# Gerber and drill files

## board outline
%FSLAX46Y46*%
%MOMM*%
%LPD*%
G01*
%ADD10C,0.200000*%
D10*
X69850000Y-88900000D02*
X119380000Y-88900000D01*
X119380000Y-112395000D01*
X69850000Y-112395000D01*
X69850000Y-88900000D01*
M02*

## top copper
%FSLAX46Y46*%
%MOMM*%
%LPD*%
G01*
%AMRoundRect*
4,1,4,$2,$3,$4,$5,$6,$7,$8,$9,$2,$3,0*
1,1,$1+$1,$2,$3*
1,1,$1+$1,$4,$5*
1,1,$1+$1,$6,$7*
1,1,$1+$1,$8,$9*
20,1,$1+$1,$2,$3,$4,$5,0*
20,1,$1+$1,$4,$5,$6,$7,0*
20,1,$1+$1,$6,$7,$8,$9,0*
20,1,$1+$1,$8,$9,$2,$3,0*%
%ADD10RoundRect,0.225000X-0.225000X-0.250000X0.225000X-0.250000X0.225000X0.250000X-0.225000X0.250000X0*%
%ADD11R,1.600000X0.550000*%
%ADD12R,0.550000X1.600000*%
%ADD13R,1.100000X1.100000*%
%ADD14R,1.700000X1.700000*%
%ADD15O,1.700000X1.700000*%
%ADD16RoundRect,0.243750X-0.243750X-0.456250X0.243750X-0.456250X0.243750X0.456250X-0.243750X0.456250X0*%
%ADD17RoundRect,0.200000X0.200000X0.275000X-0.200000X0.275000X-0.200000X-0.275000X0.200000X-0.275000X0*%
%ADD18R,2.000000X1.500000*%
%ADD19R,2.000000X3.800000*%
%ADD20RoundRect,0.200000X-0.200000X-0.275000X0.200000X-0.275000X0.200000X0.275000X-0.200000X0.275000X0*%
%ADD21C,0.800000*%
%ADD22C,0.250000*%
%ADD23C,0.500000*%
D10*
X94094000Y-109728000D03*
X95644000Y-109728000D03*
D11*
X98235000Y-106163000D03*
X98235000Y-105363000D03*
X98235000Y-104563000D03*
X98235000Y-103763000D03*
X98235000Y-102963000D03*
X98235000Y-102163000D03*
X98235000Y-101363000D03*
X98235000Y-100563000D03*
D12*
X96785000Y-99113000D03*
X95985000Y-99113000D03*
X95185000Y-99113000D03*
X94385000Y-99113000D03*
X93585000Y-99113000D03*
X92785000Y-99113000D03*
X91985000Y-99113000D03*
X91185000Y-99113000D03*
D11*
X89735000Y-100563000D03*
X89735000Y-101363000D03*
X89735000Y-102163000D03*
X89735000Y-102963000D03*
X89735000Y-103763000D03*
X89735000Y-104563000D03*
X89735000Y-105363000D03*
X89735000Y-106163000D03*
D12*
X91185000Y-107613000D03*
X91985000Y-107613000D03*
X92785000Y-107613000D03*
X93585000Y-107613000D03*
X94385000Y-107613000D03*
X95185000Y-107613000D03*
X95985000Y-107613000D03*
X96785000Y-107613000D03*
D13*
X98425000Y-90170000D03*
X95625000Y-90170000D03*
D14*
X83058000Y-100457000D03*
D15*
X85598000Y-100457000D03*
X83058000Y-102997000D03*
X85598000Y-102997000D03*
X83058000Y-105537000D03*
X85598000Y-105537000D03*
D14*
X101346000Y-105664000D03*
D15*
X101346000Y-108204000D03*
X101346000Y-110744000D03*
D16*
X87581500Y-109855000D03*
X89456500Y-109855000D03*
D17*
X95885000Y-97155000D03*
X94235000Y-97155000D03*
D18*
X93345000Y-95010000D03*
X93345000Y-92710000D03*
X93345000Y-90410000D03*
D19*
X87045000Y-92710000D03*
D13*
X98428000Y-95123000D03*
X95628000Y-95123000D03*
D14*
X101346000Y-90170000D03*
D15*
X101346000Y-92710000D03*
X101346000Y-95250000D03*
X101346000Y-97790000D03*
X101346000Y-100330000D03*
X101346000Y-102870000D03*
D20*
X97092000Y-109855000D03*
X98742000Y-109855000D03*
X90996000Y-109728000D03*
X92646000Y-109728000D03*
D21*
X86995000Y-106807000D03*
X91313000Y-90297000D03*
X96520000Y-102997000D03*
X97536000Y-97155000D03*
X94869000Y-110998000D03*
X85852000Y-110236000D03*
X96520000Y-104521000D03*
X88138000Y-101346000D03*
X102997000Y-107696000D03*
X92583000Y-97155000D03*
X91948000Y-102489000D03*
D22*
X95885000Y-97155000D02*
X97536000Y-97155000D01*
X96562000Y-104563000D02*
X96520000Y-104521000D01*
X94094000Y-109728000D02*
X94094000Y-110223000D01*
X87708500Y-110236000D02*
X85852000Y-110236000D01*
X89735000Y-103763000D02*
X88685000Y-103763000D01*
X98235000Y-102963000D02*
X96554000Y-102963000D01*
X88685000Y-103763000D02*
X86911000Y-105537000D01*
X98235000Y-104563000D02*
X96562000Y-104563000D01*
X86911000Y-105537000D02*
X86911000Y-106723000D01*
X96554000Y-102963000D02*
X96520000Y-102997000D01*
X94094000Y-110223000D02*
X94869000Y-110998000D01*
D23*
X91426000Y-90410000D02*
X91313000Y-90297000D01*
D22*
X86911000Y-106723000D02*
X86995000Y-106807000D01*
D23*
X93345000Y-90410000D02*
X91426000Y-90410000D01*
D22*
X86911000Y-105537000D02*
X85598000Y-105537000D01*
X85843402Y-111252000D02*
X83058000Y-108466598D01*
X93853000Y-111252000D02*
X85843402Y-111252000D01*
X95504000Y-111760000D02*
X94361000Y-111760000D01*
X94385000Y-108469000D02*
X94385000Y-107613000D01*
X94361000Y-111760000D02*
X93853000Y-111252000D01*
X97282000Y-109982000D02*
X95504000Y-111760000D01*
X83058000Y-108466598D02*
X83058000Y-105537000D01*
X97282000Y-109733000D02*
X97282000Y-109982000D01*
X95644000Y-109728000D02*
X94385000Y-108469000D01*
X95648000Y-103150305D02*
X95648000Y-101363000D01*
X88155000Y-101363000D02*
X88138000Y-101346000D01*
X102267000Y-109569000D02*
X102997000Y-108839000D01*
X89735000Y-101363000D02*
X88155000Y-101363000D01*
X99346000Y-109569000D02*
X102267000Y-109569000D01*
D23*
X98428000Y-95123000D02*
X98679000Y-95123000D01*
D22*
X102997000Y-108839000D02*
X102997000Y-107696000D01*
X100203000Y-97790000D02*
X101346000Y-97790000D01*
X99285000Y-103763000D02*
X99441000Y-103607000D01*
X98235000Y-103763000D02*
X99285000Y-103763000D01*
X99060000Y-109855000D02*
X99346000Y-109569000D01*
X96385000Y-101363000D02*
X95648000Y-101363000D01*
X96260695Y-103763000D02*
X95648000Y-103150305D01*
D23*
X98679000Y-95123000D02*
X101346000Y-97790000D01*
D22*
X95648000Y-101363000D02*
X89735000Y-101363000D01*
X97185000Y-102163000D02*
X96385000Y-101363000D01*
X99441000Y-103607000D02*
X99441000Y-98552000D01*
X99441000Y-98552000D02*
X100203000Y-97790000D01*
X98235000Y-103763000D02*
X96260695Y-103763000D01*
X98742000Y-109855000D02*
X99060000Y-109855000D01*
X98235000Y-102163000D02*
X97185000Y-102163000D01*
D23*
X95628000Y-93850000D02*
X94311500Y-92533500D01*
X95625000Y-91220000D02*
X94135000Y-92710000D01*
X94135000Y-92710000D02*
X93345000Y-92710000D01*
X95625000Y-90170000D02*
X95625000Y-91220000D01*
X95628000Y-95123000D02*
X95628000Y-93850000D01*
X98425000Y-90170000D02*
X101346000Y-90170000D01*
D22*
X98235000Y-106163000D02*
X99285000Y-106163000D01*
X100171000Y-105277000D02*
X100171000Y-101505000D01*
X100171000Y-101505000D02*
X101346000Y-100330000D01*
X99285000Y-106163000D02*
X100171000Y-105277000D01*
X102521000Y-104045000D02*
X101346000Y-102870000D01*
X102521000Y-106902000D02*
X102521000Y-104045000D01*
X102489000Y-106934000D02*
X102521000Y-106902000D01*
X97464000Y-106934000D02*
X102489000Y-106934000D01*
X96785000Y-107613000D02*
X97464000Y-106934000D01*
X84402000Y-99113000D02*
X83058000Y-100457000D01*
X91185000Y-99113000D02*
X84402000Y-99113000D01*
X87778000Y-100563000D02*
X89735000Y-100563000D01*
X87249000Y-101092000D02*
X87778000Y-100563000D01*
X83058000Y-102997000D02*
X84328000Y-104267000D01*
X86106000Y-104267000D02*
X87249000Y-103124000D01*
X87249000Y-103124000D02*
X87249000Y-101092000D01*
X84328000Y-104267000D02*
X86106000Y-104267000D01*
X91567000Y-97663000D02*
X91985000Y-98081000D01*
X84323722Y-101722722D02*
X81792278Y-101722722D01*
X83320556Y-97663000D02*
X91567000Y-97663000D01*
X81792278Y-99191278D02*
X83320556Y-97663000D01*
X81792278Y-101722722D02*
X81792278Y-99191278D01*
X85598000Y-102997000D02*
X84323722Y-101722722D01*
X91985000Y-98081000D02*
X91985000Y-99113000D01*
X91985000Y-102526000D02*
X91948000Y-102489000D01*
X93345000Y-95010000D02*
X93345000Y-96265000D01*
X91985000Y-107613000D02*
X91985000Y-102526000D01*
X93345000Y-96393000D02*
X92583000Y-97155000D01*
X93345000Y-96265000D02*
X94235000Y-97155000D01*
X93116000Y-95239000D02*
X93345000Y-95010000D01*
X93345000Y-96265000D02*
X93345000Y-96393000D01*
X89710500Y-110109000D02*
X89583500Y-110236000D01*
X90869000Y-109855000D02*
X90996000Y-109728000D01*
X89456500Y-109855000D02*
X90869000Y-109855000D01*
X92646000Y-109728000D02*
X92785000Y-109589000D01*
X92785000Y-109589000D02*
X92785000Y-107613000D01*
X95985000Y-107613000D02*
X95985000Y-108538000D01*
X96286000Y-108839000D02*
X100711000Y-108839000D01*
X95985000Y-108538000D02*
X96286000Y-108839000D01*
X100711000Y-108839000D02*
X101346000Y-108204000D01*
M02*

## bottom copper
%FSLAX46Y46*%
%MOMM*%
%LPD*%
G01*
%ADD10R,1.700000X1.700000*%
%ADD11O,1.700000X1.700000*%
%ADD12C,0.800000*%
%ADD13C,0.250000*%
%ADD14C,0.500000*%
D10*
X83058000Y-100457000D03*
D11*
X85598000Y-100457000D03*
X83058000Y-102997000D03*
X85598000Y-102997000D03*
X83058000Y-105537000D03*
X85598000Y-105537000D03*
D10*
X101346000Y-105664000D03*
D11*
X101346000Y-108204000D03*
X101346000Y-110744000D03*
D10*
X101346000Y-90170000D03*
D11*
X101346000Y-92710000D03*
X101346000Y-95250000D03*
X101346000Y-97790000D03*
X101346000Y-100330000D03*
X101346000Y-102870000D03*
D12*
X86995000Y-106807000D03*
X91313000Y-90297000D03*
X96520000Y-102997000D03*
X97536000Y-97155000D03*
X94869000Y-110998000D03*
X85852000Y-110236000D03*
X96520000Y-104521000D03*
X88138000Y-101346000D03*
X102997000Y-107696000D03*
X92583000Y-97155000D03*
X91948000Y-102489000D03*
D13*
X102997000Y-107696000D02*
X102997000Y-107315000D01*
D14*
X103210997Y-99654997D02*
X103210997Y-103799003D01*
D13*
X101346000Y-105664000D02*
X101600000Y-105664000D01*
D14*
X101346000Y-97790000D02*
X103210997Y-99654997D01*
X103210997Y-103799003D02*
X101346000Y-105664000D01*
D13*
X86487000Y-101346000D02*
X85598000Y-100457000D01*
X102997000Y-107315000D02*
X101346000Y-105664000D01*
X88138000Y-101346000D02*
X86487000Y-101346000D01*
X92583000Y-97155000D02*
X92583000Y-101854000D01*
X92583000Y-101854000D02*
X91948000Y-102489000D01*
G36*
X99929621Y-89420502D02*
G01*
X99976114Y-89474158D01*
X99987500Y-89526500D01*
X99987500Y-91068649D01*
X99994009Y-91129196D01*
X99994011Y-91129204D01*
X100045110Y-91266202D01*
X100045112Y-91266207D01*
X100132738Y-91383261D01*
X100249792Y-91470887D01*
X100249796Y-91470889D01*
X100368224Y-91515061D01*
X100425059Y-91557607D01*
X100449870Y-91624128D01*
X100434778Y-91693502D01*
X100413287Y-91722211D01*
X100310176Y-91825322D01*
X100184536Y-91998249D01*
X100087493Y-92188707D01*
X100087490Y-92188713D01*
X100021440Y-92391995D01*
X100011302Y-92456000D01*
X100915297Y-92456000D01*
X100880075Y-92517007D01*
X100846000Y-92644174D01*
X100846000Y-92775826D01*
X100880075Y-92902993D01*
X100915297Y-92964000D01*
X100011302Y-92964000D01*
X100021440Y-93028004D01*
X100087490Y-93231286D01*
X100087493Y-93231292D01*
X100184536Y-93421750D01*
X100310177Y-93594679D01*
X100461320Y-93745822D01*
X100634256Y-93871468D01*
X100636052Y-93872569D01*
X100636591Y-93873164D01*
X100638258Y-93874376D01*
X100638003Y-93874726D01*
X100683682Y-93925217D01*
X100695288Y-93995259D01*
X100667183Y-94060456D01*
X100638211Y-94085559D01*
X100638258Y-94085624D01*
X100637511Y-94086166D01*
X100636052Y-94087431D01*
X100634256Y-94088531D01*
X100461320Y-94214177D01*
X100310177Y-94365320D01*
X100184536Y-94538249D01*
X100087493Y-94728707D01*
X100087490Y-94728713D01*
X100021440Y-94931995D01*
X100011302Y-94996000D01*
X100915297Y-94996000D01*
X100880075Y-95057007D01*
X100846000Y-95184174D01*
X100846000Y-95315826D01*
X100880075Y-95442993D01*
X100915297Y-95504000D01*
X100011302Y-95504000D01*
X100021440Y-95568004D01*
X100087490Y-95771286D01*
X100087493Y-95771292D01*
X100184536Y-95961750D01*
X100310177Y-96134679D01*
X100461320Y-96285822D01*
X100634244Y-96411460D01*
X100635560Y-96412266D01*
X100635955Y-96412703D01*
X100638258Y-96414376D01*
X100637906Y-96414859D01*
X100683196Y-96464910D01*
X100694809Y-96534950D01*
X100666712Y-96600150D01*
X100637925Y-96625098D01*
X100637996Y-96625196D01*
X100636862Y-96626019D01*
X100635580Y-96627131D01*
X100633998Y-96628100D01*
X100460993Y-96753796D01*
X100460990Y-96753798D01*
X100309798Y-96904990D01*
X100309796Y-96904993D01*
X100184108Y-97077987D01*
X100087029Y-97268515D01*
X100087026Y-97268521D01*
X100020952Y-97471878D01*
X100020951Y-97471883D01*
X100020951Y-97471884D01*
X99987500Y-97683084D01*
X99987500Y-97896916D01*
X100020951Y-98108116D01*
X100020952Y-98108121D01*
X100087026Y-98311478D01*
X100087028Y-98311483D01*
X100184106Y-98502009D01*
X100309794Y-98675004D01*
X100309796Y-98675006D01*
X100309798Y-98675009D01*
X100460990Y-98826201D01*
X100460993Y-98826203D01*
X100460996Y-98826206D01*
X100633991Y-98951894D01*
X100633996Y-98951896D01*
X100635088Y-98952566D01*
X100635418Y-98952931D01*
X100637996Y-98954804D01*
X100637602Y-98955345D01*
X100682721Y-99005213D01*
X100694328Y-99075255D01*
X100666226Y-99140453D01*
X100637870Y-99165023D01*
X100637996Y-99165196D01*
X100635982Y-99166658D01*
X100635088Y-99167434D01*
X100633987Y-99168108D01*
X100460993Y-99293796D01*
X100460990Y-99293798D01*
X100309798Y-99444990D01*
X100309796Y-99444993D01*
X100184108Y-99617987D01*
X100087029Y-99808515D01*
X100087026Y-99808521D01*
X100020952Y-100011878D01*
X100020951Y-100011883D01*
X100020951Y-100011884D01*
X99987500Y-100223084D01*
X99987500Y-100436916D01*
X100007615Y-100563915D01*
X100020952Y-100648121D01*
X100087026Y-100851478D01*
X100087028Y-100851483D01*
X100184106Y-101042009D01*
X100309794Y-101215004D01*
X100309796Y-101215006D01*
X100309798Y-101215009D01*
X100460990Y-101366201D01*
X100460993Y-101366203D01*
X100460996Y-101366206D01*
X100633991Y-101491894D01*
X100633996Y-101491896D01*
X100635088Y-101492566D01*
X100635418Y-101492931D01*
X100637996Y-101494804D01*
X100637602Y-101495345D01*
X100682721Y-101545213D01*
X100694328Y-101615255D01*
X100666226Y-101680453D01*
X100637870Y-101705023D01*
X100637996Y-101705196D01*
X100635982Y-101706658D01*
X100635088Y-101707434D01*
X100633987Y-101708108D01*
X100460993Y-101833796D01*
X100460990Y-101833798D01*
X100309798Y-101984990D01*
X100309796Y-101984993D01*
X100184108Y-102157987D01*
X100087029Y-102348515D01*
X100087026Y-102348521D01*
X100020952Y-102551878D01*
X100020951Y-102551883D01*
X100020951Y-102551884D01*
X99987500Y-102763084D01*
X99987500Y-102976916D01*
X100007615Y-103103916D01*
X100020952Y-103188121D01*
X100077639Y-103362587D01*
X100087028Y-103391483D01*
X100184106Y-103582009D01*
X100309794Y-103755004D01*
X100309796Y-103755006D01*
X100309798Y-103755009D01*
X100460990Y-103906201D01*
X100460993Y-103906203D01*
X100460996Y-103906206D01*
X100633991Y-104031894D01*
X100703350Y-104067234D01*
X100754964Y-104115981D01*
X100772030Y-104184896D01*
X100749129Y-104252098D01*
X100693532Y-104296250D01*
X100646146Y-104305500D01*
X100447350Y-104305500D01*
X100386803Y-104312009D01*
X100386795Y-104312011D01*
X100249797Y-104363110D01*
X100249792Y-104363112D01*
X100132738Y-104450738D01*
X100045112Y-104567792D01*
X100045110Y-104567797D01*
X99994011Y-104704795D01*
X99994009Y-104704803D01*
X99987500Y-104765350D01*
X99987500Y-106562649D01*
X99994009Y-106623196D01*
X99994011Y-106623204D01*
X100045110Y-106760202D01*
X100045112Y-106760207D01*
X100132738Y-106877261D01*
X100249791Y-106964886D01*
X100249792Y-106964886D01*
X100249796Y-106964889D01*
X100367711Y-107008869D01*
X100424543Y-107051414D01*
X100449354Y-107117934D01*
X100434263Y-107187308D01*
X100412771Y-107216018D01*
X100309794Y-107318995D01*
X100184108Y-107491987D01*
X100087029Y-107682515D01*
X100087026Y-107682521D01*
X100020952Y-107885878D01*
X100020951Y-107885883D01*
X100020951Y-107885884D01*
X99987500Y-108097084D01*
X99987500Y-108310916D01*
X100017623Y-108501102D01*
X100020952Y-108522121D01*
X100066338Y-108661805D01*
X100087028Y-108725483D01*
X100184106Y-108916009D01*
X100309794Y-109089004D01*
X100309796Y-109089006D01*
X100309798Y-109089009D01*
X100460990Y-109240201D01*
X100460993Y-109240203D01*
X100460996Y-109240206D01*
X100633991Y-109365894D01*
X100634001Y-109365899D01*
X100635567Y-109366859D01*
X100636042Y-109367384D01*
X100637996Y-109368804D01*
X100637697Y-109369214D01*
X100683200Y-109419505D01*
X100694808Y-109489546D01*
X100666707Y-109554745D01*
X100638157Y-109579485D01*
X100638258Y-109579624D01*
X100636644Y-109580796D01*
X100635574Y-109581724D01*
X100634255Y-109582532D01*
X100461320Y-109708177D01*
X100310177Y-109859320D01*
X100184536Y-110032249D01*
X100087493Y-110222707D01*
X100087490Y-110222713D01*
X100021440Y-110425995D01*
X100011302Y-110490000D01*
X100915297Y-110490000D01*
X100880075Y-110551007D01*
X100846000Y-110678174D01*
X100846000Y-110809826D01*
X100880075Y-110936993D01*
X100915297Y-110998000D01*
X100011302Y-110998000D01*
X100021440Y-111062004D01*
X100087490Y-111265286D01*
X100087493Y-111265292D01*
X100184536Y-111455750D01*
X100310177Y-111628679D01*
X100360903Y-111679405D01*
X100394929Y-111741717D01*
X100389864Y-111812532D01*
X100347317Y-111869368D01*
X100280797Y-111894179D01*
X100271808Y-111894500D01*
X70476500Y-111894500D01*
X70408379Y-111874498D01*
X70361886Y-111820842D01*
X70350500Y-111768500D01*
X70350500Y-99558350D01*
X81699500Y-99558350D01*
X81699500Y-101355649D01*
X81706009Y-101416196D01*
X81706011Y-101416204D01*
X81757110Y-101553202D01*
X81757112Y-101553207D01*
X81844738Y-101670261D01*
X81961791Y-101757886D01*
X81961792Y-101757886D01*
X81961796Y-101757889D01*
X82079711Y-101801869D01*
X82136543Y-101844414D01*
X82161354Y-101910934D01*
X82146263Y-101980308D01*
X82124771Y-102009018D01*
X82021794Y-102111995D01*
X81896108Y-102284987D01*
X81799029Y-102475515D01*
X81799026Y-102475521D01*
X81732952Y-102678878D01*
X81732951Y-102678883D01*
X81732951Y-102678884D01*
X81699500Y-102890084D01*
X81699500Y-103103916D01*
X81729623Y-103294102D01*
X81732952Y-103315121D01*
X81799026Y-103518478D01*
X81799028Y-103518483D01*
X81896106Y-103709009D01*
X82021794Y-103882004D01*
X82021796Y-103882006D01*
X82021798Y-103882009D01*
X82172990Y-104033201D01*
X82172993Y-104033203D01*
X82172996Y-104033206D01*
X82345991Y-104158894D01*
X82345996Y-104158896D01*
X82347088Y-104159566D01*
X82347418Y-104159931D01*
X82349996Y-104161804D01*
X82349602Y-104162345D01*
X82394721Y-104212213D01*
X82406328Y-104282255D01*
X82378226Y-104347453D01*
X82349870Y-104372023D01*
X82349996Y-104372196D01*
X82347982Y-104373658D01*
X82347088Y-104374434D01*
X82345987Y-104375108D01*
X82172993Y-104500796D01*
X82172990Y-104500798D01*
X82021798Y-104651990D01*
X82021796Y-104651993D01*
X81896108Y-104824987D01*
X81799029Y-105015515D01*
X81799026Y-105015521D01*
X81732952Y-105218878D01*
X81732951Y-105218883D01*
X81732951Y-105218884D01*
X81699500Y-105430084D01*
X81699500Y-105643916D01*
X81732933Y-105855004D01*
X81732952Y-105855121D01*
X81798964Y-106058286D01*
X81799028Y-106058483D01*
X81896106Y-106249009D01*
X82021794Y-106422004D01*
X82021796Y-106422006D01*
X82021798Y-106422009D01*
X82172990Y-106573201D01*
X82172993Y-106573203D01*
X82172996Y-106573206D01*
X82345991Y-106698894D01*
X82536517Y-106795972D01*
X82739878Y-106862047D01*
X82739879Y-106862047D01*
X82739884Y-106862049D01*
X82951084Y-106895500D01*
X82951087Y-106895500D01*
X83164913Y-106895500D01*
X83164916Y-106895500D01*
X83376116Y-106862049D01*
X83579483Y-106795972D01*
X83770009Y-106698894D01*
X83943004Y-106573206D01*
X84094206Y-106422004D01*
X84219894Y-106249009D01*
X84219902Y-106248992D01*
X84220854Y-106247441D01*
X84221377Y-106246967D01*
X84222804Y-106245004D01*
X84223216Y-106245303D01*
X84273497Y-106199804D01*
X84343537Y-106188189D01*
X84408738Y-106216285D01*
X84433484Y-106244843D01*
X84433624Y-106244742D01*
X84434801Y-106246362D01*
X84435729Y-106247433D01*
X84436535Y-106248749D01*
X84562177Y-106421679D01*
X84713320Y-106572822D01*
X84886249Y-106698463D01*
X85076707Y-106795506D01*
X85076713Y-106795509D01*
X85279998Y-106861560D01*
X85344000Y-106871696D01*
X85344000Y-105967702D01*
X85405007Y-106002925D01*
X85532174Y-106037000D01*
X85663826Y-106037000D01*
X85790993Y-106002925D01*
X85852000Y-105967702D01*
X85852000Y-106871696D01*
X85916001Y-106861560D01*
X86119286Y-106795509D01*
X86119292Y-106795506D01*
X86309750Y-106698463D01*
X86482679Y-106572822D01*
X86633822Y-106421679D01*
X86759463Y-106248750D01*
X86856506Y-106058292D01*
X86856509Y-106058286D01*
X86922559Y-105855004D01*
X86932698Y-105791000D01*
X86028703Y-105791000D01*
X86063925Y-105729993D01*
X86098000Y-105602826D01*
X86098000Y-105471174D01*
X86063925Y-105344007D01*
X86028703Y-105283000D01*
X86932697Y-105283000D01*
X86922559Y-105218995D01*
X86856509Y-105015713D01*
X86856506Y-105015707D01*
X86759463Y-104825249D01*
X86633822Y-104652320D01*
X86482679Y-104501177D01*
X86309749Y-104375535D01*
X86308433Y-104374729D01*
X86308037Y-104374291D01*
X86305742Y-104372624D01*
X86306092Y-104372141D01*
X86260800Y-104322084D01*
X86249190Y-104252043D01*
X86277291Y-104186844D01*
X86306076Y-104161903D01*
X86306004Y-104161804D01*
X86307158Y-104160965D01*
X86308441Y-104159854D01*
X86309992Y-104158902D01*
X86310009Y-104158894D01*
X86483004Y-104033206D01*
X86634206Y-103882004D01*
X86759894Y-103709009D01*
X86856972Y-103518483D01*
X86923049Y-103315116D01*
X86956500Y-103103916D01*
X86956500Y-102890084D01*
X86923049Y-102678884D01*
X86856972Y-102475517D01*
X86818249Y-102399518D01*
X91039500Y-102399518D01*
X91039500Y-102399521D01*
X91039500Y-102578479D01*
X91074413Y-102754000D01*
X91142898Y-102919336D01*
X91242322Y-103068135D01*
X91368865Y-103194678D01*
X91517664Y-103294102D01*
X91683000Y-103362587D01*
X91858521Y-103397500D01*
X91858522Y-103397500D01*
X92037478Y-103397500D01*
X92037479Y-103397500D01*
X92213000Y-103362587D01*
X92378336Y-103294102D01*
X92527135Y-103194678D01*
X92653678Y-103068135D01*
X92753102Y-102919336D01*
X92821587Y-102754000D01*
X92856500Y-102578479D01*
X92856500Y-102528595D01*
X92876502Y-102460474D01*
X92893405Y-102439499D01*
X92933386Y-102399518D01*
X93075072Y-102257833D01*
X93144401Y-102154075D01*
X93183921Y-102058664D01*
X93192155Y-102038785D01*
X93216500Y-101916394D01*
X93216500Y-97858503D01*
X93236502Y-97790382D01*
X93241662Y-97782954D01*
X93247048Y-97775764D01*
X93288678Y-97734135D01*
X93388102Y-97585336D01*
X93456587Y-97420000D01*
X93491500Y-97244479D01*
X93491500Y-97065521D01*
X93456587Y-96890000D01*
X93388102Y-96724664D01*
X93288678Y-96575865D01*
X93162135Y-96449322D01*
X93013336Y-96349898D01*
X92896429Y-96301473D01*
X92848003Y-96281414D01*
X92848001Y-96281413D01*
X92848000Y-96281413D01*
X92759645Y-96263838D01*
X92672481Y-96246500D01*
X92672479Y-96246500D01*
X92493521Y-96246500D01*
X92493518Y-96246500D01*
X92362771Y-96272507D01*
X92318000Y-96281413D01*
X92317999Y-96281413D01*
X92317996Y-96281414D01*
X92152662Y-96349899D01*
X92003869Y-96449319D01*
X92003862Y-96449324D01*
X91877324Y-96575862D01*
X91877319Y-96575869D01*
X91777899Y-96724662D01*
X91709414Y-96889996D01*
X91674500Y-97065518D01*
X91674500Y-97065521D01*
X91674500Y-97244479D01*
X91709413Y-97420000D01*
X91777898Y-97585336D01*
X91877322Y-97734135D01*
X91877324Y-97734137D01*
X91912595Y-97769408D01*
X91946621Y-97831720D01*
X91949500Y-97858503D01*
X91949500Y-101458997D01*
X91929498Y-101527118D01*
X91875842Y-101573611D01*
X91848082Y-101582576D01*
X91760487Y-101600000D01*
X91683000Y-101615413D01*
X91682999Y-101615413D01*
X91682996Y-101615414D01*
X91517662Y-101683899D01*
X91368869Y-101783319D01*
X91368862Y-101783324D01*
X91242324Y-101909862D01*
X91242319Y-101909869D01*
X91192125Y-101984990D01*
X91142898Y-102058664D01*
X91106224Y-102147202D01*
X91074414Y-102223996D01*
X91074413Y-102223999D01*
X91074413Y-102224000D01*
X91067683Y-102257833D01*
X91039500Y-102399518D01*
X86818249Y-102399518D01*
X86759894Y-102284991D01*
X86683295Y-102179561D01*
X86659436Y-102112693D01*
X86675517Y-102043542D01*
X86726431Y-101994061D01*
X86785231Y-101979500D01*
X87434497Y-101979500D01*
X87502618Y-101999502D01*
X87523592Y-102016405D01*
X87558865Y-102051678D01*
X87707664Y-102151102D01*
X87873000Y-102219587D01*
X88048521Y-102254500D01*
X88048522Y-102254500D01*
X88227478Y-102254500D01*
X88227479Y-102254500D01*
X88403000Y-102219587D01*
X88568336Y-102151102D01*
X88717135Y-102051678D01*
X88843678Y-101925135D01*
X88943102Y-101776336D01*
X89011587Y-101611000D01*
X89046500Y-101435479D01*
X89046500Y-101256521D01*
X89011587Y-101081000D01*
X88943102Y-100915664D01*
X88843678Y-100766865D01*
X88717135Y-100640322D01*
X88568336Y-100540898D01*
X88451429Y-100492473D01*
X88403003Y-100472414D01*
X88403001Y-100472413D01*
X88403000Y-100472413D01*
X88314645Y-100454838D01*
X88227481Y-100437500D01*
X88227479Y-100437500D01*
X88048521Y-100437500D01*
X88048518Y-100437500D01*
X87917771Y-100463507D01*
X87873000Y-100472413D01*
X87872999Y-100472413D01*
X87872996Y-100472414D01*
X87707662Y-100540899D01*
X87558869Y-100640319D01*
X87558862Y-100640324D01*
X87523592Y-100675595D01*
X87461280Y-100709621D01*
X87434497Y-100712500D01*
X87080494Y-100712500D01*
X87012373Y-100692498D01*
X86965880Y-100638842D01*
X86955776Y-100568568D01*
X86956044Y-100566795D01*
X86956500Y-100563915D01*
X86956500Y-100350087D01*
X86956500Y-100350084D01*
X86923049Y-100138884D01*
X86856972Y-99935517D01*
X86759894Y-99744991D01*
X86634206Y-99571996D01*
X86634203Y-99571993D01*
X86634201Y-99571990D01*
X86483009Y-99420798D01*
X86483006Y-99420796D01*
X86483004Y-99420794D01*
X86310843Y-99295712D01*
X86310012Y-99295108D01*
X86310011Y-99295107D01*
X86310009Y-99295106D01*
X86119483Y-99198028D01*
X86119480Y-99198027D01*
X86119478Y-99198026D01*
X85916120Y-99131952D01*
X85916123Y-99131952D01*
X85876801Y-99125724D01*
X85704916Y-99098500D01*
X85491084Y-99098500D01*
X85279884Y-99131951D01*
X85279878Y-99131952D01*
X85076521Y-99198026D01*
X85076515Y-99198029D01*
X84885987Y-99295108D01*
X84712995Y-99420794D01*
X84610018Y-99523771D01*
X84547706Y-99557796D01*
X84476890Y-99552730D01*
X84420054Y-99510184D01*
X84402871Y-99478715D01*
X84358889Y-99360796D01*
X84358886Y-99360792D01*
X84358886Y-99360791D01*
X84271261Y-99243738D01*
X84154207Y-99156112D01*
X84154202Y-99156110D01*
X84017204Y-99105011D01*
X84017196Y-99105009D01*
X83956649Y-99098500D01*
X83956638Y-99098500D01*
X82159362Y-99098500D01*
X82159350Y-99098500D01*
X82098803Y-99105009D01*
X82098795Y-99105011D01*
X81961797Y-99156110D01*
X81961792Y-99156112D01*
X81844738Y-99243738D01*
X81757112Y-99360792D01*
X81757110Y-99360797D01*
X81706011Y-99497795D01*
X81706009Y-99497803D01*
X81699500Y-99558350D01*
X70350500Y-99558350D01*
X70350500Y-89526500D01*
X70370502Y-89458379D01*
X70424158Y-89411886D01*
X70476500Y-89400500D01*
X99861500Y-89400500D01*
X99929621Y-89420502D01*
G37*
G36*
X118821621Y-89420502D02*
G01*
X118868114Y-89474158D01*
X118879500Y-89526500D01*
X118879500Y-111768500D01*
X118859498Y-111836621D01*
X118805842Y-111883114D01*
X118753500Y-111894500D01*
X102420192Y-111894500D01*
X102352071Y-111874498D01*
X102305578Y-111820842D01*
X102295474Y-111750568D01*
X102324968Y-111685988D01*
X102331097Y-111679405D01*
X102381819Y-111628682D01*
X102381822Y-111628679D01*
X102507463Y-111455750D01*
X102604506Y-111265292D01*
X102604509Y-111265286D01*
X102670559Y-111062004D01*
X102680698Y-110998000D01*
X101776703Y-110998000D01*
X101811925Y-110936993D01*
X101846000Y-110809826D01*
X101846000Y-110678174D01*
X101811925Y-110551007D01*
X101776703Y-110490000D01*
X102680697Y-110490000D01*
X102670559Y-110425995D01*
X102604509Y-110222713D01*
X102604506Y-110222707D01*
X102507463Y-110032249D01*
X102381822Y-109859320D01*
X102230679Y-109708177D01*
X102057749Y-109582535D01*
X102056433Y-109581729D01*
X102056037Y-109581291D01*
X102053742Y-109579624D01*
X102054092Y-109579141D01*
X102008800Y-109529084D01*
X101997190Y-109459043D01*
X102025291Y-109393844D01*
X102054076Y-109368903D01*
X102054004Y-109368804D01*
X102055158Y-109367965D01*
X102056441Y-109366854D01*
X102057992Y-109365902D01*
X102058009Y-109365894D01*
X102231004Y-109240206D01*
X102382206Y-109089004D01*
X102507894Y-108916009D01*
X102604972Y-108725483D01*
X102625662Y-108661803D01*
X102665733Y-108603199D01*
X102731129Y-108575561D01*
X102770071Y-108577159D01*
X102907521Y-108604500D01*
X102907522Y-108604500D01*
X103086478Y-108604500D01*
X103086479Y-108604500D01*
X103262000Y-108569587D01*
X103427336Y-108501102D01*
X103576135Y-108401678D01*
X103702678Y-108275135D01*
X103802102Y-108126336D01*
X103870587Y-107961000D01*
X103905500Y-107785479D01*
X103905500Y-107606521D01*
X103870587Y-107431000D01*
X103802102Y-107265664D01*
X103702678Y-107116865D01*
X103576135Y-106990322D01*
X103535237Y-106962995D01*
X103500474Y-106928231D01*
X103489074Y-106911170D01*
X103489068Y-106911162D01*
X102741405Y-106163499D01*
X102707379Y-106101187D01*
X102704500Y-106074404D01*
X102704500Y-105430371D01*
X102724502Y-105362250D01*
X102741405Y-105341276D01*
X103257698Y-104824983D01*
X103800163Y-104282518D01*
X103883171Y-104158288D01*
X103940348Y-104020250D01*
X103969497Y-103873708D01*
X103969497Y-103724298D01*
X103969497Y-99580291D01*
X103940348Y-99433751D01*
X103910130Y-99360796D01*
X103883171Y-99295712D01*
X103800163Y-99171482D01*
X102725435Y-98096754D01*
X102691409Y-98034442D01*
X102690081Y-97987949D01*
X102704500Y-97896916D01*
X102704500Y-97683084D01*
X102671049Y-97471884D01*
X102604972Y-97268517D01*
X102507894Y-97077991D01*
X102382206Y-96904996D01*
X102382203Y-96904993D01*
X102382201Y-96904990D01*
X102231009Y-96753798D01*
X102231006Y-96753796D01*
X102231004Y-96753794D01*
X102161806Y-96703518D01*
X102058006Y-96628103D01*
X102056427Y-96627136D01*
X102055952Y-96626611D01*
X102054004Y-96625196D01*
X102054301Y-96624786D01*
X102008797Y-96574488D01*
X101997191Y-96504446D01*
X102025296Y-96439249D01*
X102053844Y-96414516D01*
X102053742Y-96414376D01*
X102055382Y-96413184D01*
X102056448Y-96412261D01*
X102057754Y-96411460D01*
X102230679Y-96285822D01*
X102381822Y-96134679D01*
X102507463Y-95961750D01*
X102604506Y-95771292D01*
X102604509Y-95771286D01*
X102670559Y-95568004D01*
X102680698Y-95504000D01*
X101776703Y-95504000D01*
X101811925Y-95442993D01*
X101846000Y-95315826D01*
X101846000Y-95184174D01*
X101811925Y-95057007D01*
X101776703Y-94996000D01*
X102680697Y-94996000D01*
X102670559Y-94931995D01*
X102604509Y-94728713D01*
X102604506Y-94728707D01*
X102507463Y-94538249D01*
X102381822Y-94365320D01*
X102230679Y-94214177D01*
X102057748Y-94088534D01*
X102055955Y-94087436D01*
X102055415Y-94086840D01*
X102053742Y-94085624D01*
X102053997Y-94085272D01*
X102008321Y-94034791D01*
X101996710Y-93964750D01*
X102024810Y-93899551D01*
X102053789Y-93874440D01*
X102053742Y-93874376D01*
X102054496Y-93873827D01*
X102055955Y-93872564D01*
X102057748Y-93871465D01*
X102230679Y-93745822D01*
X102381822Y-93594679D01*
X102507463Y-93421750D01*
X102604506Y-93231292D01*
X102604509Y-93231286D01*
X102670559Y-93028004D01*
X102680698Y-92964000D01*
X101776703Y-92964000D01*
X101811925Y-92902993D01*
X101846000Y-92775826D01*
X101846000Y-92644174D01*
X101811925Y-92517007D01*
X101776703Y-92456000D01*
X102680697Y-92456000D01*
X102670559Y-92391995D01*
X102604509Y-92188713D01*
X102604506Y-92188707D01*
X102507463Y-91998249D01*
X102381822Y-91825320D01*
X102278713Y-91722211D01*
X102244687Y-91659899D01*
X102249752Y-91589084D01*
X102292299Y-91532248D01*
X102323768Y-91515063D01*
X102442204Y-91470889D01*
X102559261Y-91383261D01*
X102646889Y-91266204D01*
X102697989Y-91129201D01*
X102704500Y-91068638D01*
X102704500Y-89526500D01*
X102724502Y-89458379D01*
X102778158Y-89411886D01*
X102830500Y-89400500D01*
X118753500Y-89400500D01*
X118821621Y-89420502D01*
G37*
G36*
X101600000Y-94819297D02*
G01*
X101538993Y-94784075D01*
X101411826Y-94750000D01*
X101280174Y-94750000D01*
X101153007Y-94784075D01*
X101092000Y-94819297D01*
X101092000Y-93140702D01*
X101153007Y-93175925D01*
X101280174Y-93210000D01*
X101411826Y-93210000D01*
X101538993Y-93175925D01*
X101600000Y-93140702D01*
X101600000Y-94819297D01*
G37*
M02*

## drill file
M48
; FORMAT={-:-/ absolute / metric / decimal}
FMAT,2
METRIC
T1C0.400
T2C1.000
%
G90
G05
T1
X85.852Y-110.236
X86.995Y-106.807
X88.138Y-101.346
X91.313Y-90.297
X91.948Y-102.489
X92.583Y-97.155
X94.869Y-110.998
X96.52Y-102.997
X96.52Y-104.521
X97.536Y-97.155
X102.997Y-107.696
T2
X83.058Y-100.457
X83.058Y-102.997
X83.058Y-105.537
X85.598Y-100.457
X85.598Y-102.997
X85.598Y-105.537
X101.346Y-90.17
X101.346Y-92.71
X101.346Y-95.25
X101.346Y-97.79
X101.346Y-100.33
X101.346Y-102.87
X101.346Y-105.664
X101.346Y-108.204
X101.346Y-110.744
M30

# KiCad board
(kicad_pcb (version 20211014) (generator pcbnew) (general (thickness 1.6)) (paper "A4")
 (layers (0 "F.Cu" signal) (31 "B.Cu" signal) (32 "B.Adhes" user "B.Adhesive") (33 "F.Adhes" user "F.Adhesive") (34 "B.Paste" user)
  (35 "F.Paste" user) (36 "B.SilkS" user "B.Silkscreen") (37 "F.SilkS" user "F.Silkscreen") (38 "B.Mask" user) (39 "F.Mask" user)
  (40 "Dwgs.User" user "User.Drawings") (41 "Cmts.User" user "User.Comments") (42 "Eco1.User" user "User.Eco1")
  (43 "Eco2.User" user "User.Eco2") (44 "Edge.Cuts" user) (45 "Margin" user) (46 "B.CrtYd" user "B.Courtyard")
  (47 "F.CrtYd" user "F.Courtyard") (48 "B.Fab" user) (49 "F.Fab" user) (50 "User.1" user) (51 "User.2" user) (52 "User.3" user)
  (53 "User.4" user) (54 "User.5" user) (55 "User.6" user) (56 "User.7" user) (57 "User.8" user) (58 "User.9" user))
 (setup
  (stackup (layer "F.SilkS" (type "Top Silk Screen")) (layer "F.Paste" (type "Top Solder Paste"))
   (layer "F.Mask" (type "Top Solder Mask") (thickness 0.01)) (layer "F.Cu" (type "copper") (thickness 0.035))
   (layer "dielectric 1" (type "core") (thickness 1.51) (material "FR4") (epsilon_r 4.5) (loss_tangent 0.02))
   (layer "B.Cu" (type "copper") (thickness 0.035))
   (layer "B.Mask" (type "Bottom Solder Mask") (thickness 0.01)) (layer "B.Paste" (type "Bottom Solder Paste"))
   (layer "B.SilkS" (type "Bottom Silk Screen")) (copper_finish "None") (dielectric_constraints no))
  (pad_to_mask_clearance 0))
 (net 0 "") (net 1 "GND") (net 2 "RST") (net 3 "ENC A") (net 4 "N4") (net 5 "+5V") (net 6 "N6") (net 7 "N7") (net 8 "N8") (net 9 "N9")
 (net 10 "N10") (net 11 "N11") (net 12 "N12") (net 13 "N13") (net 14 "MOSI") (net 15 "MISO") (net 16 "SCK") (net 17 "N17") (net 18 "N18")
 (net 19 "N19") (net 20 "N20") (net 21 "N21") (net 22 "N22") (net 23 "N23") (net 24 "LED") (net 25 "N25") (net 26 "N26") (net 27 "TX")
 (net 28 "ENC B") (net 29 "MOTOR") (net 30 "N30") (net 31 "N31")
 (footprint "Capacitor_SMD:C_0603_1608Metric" (layer "F.Cu") (at 94.869 109.728)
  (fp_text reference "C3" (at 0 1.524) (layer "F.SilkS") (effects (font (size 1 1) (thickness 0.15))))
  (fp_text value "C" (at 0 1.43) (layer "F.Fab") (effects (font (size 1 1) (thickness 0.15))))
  (pad "1" smd roundrect (at -0.775 0) (size 0.9 0.95) (layers "F.Cu" "F.Paste" "F.Mask") (roundrect_rratio 0.25) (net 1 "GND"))
  (pad "2" smd roundrect (at 0.775 0) (size 0.9 0.95) (layers "F.Cu" "F.Paste" "F.Mask") (roundrect_rratio 0.25) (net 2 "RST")))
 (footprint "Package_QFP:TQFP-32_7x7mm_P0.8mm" (layer "F.Cu") (at 93.985 103.363 180)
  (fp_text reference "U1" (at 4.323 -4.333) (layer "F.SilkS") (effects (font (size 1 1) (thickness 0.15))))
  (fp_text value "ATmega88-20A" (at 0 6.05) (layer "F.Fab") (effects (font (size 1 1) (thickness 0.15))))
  (pad "1" smd rect (at -4.25 -2.8 180) (size 1.6 0.55) (layers "F.Cu" "F.Paste" "F.Mask") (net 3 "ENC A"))
  (pad "2" smd rect (at -4.25 -2 180) (size 1.6 0.55) (layers "F.Cu" "F.Paste" "F.Mask") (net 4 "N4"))
  (pad "3" smd rect (at -4.25 -1.2 180) (size 1.6 0.55) (layers "F.Cu" "F.Paste" "F.Mask") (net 1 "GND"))
  (pad "4" smd rect (at -4.25 -0.4 180) (size 1.6 0.55) (layers "F.Cu" "F.Paste" "F.Mask") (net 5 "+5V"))
  (pad "5" smd rect (at -4.25 0.4 180) (size 1.6 0.55) (layers "F.Cu" "F.Paste" "F.Mask") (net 1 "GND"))
  (pad "6" smd rect (at -4.25 1.2 180) (size 1.6 0.55) (layers "F.Cu" "F.Paste" "F.Mask") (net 5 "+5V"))
  (pad "7" smd rect (at -4.25 2 180) (size 1.6 0.55) (layers "F.Cu" "F.Paste" "F.Mask") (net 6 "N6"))
  (pad "8" smd rect (at -4.25 2.8 180) (size 1.6 0.55) (layers "F.Cu" "F.Paste" "F.Mask") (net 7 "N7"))
  (pad "9" smd rect (at -2.8 4.25 270) (size 1.6 0.55) (layers "F.Cu" "F.Paste" "F.Mask") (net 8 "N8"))
  (pad "10" smd rect (at -2 4.25 270) (size 1.6 0.55) (layers "F.Cu" "F.Paste" "F.Mask") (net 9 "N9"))
  (pad "11" smd rect (at -1.2 4.25 270) (size 1.6 0.55) (layers "F.Cu" "F.Paste" "F.Mask") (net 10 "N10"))
  (pad "12" smd rect (at -0.4 4.25 270) (size 1.6 0.55) (layers "F.Cu" "F.Paste" "F.Mask") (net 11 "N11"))
  (pad "13" smd rect (at 0.4 4.25 270) (size 1.6 0.55) (layers "F.Cu" "F.Paste" "F.Mask") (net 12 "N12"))
  (pad "14" smd rect (at 1.2 4.25 270) (size 1.6 0.55) (layers "F.Cu" "F.Paste" "F.Mask") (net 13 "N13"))
  (pad "15" smd rect (at 2 4.25 270) (size 1.6 0.55) (layers "F.Cu" "F.Paste" "F.Mask") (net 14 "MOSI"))
  (pad "16" smd rect (at 2.8 4.25 270) (size 1.6 0.55) (layers "F.Cu" "F.Paste" "F.Mask") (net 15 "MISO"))
  (pad "17" smd rect (at 4.25 2.8 180) (size 1.6 0.55) (layers "F.Cu" "F.Paste" "F.Mask") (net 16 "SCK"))
  (pad "18" smd rect (at 4.25 2 180) (size 1.6 0.55) (layers "F.Cu" "F.Paste" "F.Mask") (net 5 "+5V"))
  (pad "19" smd rect (at 4.25 1.2 180) (size 1.6 0.55) (layers "F.Cu" "F.Paste" "F.Mask") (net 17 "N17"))
  (pad "20" smd rect (at 4.25 0.4 180) (size 1.6 0.55) (layers "F.Cu" "F.Paste" "F.Mask") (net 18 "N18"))
  (pad "21" smd rect (at 4.25 -0.4 180) (size 1.6 0.55) (layers "F.Cu" "F.Paste" "F.Mask") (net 1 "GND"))
  (pad "22" smd rect (at 4.25 -1.2 180) (size 1.6 0.55) (layers "F.Cu" "F.Paste" "F.Mask") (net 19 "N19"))
  (pad "23" smd rect (at 4.25 -2 180) (size 1.6 0.55) (layers "F.Cu" "F.Paste" "F.Mask") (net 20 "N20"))
  (pad "24" smd rect (at 4.25 -2.8 180) (size 1.6 0.55) (layers "F.Cu" "F.Paste" "F.Mask") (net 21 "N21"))
  (pad "25" smd rect (at 2.8 -4.25 270) (size 1.6 0.55) (layers "F.Cu" "F.Paste" "F.Mask") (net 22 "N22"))
  (pad "26" smd rect (at 2 -4.25 270) (size 1.6 0.55) (layers "F.Cu" "F.Paste" "F.Mask") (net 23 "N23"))
  (pad "27" smd rect (at 1.2 -4.25 270) (size 1.6 0.55) (layers "F.Cu" "F.Paste" "F.Mask") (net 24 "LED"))
  (pad "28" smd rect (at 0.4 -4.25 270) (size 1.6 0.55) (layers "F.Cu" "F.Paste" "F.Mask") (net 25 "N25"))
  (pad "29" smd rect (at -0.4 -4.25 270) (size 1.6 0.55) (layers "F.Cu" "F.Paste" "F.Mask") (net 2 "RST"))
  (pad "30" smd rect (at -1.2 -4.25 270) (size 1.6 0.55) (layers "F.Cu" "F.Paste" "F.Mask") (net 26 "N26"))
  (pad "31" smd rect (at -2 -4.25 270) (size 1.6 0.55) (layers "F.Cu" "F.Paste" "F.Mask") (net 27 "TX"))
  (pad "32" smd rect (at -2.8 -4.25 270) (size 1.6 0.55) (layers "F.Cu" "F.Paste" "F.Mask") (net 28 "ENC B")))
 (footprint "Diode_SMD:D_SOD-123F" (layer "F.Cu") (at 97.025 90.17 180)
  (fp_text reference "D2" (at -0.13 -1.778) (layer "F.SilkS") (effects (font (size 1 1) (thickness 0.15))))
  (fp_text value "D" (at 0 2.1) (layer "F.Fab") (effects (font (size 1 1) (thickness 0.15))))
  (pad "1" smd rect (at -1.4 0 180) (size 1.1 1.1) (layers "F.Cu" "F.Paste" "F.Mask") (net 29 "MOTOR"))
  (pad "2" smd rect (at 1.4 0 180) (size 1.1 1.1) (layers "F.Cu" "F.Paste" "F.Mask") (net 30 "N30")))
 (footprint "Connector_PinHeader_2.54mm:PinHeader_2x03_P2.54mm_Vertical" (layer "F.Cu") (at 83.058 100.457)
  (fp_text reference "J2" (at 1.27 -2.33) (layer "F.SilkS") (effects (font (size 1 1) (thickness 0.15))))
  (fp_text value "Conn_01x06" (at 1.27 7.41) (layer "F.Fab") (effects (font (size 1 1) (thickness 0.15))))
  (pad "1" thru_hole rect (at 0 0) (size 1.7 1.7) (drill 1) (layers *.Cu *.Mask) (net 15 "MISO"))
  (pad "2" thru_hole oval (at 2.54 0) (size 1.7 1.7) (drill 1) (layers *.Cu *.Mask) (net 5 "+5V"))
  (pad "3" thru_hole oval (at 0 2.54) (size 1.7 1.7) (drill 1) (layers *.Cu *.Mask) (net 16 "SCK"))
  (pad "4" thru_hole oval (at 2.54 2.54) (size 1.7 1.7) (drill 1) (layers *.Cu *.Mask) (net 14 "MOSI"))
  (pad "5" thru_hole oval (at 0 5.08) (size 1.7 1.7) (drill 1) (layers *.Cu *.Mask) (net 2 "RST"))
  (pad "6" thru_hole oval (at 2.54 5.08) (size 1.7 1.7) (drill 1) (layers *.Cu *.Mask) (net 1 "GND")))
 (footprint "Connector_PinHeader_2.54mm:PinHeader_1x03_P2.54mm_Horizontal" (layer "F.Cu") (at 101.346 105.664)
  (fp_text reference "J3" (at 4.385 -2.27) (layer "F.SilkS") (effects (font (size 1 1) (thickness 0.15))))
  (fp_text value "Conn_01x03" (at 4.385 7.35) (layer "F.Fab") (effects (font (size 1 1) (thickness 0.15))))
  (pad "1" thru_hole rect (at 0 0) (size 1.7 1.7) (drill 1) (layers *.Cu *.Mask) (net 5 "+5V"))
  (pad "2" thru_hole oval (at 0 2.54) (size 1.7 1.7) (drill 1) (layers *.Cu *.Mask) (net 27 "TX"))
  (pad "3" thru_hole oval (at 0 5.08) (size 1.7 1.7) (drill 1) (layers *.Cu *.Mask) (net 1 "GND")))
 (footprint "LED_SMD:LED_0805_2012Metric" (layer "F.Cu") (at 88.519 109.855)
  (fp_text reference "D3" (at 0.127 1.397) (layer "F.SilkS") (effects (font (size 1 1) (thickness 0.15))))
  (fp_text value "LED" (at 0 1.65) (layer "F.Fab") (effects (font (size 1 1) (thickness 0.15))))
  (pad "1" smd roundrect (at -0.9375 0) (size 0.975 1.4) (layers "F.Cu" "F.Paste" "F.Mask") (roundrect_rratio 0.25) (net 1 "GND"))
  (pad "2" smd roundrect (at 0.9375 0) (size 0.975 1.4) (layers "F.Cu" "F.Paste" "F.Mask") (roundrect_rratio 0.25) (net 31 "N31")))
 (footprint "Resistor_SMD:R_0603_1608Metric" (layer "F.Cu") (at 95.06 97.155 180)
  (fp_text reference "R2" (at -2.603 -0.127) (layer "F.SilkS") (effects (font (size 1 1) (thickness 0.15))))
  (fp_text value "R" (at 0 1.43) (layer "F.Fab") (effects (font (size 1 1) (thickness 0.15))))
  (pad "1" smd roundrect (at -0.825 0 180) (size 0.8 0.95) (layers "F.Cu" "F.Paste" "F.Mask") (roundrect_rratio 0.25) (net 1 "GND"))
  (pad "2" smd roundrect (at 0.825 0 180) (size 0.8 0.95) (layers "F.Cu" "F.Paste" "F.Mask") (roundrect_rratio 0.25) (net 23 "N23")))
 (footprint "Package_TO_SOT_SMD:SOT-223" (layer "F.Cu") (at 90.195 92.71 180)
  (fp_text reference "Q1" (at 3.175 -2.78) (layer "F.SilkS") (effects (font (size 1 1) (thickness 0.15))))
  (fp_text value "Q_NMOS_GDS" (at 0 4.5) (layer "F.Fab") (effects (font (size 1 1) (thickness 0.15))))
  (pad "1" smd rect (at -3.15 -2.3 180) (size 2 1.5) (layers "F.Cu" "F.Paste" "F.Mask") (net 23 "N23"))
  (pad "2" smd rect (at -3.15 0 180) (size 2 1.5) (layers "F.Cu" "F.Paste" "F.Mask") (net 30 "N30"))
  (pad "3" smd rect (at -3.15 2.3 180) (size 2 1.5) (layers "F.Cu" "F.Paste" "F.Mask") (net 1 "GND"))
  (pad "4" smd rect (at 3.15 0 180) (size 2 3.8) (layers "F.Cu" "F.Paste" "F.Mask")))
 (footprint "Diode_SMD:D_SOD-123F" (layer "F.Cu") (at 97.028 95.123 180)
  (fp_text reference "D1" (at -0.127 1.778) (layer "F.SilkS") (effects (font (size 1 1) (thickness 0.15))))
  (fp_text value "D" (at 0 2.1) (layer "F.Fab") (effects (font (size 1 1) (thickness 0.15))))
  (pad "1" smd rect (at -1.4 0 180) (size 1.1 1.1) (layers "F.Cu" "F.Paste" "F.Mask") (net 5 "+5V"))
  (pad "2" smd rect (at 1.4 0 180) (size 1.1 1.1) (layers "F.Cu" "F.Paste" "F.Mask") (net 30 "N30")))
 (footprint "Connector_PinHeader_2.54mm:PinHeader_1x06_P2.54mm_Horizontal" (layer "F.Cu") (at 101.346 90.17)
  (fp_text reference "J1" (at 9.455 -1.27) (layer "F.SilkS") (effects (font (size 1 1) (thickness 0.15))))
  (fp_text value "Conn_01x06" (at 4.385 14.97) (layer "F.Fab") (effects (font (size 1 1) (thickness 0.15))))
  (pad "1" thru_hole rect (at 0 0) (size 1.7 1.7) (drill 1) (layers *.Cu *.Mask) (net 29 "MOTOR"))
  (pad "2" thru_hole oval (at 0 2.54) (size 1.7 1.7) (drill 1) (layers *.Cu *.Mask) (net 1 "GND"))
  (pad "3" thru_hole oval (at 0 5.08) (size 1.7 1.7) (drill 1) (layers *.Cu *.Mask) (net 1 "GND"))
  (pad "4" thru_hole oval (at 0 7.62) (size 1.7 1.7) (drill 1) (layers *.Cu *.Mask) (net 5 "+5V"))
  (pad "5" thru_hole oval (at 0 10.16) (size 1.7 1.7) (drill 1) (layers *.Cu *.Mask) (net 3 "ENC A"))
  (pad "6" thru_hole oval (at 0 12.7) (size 1.7 1.7) (drill 1) (layers *.Cu *.Mask) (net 28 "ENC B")))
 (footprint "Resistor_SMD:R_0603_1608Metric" (layer "F.Cu") (at 97.917 109.855)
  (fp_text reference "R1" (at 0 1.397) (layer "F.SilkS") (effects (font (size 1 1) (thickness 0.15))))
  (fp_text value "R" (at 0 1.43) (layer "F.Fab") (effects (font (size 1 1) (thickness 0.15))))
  (pad "1" smd roundrect (at -0.825 0) (size 0.8 0.95) (layers "F.Cu" "F.Paste" "F.Mask") (roundrect_rratio 0.25) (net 2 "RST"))
  (pad "2" smd roundrect (at 0.825 0) (size 0.8 0.95) (layers "F.Cu" "F.Paste" "F.Mask") (roundrect_rratio 0.25) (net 5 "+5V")))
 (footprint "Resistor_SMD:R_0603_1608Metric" (layer "F.Cu") (at 91.821 109.728)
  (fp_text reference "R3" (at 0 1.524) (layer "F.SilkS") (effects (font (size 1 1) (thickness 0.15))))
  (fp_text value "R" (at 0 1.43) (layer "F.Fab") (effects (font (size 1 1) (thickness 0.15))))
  (pad "1" smd roundrect (at -0.825 0) (size 0.8 0.95) (layers "F.Cu" "F.Paste" "F.Mask") (roundrect_rratio 0.25) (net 31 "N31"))
  (pad "2" smd roundrect (at 0.825 0) (size 0.8 0.95) (layers "F.Cu" "F.Paste" "F.Mask") (roundrect_rratio 0.25) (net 24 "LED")))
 (gr_rect (start 69.85 88.9) (end 119.38 112.395) (layer "Edge.Cuts") (width 0.2) (fill none))
 (segment (start 95.885 97.155) (end 97.536 97.155) (width 0.25) (layer "F.Cu") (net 1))
 (segment (start 96.562 104.563) (end 96.52 104.521) (width 0.25) (layer "F.Cu") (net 1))
 (segment (start 94.094 109.728) (end 94.094 110.223) (width 0.25) (layer "F.Cu") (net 1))
 (segment (start 87.7085 110.236) (end 85.852 110.236) (width 0.25) (layer "F.Cu") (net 1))
 (segment (start 89.735 103.763) (end 88.685 103.763) (width 0.25) (layer "F.Cu") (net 1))
 (segment (start 98.235 102.963) (end 96.554 102.963) (width 0.25) (layer "F.Cu") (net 1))
 (segment (start 88.685 103.763) (end 86.911 105.537) (width 0.25) (layer "F.Cu") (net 1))
 (segment (start 98.235 104.563) (end 96.562 104.563) (width 0.25) (layer "F.Cu") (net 1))
 (segment (start 86.911 105.537) (end 86.911 106.723) (width 0.25) (layer "F.Cu") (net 1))
 (segment (start 96.554 102.963) (end 96.52 102.997) (width 0.25) (layer "F.Cu") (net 1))
 (segment (start 94.094 110.223) (end 94.869 110.998) (width 0.25) (layer "F.Cu") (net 1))
 (segment (start 91.426 90.41) (end 91.313 90.297) (width 0.5) (layer "F.Cu") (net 1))
 (segment (start 86.911 106.723) (end 86.995 106.807) (width 0.25) (layer "F.Cu") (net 1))
 (segment (start 93.345 90.41) (end 91.426 90.41) (width 0.5) (layer "F.Cu") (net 1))
 (segment (start 86.911 105.537) (end 85.598 105.537) (width 0.25) (layer "F.Cu") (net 1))
 (via (at 86.995 106.807) (size 0.8) (drill 0.4) (layers "F.Cu" "B.Cu") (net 1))
 (via (at 91.313 90.297) (size 0.8) (drill 0.4) (layers "F.Cu" "B.Cu") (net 1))
 (via (at 96.52 102.997) (size 0.8) (drill 0.4) (layers "F.Cu" "B.Cu") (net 1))
 (via (at 97.536 97.155) (size 0.8) (drill 0.4) (layers "F.Cu" "B.Cu") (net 1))
 (via (at 94.869 110.998) (size 0.8) (drill 0.4) (layers "F.Cu" "B.Cu") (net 1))
 (via (at 85.852 110.236) (size 0.8) (drill 0.4) (layers "F.Cu" "B.Cu") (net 1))
 (via (at 96.52 104.521) (size 0.8) (drill 0.4) (layers "F.Cu" "B.Cu") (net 1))
 (segment (start 85.843402 111.252) (end 83.058 108.466598) (width 0.25) (layer "F.Cu") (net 2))
 (segment (start 93.853 111.252) (end 85.843402 111.252) (width 0.25) (layer "F.Cu") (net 2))
 (segment (start 95.504 111.76) (end 94.361 111.76) (width 0.25) (layer "F.Cu") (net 2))
 (segment (start 94.385 108.469) (end 94.385 107.613) (width 0.25) (layer "F.Cu") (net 2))
 (segment (start 94.361 111.76) (end 93.853 111.252) (width 0.25) (layer "F.Cu") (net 2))
 (segment (start 97.282 109.982) (end 95.504 111.76) (width 0.25) (layer "F.Cu") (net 2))
 (segment (start 83.058 108.466598) (end 83.058 105.537) (width 0.25) (layer "F.Cu") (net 2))
 (segment (start 97.282 109.733) (end 97.282 109.982) (width 0.25) (layer "F.Cu") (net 2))
 (segment (start 95.644 109.728) (end 94.385 108.469) (width 0.25) (layer "F.Cu") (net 2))
 (segment (start 95.648 103.150305) (end 95.648 101.363) (width 0.25) (layer "F.Cu") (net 5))
 (segment (start 88.155 101.363) (end 88.138 101.346) (width 0.25) (layer "F.Cu") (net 5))
 (segment (start 102.267 109.569) (end 102.997 108.839) (width 0.25) (layer "F.Cu") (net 5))
 (segment (start 89.735 101.363) (end 88.155 101.363) (width 0.25) (layer "F.Cu") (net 5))
 (segment (start 99.346 109.569) (end 102.267 109.569) (width 0.25) (layer "F.Cu") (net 5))
 (segment (start 98.428 95.123) (end 98.679 95.123) (width 0.5) (layer "F.Cu") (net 5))
 (segment (start 102.997 108.839) (end 102.997 107.696) (width 0.25) (layer "F.Cu") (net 5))
 (segment (start 100.203 97.79) (end 101.346 97.79) (width 0.25) (layer "F.Cu") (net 5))
 (segment (start 99.285 103.763) (end 99.441 103.607) (width 0.25) (layer "F.Cu") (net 5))
 (segment (start 98.235 103.763) (end 99.285 103.763) (width 0.25) (layer "F.Cu") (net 5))
 (segment (start 99.06 109.855) (end 99.346 109.569) (width 0.25) (layer "F.Cu") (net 5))
 (segment (start 96.385 101.363) (end 95.648 101.363) (width 0.25) (layer "F.Cu") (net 5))
 (segment (start 96.260695 103.763) (end 95.648 103.150305) (width 0.25) (layer "F.Cu") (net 5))
 (segment (start 98.679 95.123) (end 101.346 97.79) (width 0.5) (layer "F.Cu") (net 5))
 (segment (start 95.648 101.363) (end 89.735 101.363) (width 0.25) (layer "F.Cu") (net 5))
 (segment (start 97.185 102.163) (end 96.385 101.363) (width 0.25) (layer "F.Cu") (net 5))
 (segment (start 99.441 103.607) (end 99.441 98.552) (width 0.25) (layer "F.Cu") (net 5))
 (segment (start 99.441 98.552) (end 100.203 97.79) (width 0.25) (layer "F.Cu") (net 5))
 (segment (start 98.235 103.763) (end 96.260695 103.763) (width 0.25) (layer "F.Cu") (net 5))
 (segment (start 98.742 109.855) (end 99.06 109.855) (width 0.25) (layer "F.Cu") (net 5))
 (segment (start 98.235 102.163) (end 97.185 102.163) (width 0.25) (layer "F.Cu") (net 5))
 (via (at 88.138 101.346) (size 0.8) (drill 0.4) (layers "F.Cu" "B.Cu") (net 5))
 (via (at 102.997 107.696) (size 0.8) (drill 0.4) (layers "F.Cu" "B.Cu") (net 5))
 (segment (start 102.997 107.696) (end 102.997 107.315) (width 0.25) (layer "B.Cu") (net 5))
 (segment (start 103.210997 99.654997) (end 103.210997 103.799003) (width 0.5) (layer "B.Cu") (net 5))
 (segment (start 101.346 105.664) (end 101.6 105.664) (width 0.25) (layer "B.Cu") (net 5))
 (segment (start 101.346 97.79) (end 103.210997 99.654997) (width 0.5) (layer "B.Cu") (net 5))
 (segment (start 103.210997 103.799003) (end 101.346 105.664) (width 0.5) (layer "B.Cu") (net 5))
 (segment (start 86.487 101.346) (end 85.598 100.457) (width 0.25) (layer "B.Cu") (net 5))
 (segment (start 102.997 107.315) (end 101.346 105.664) (width 0.25) (layer "B.Cu") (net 5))
 (segment (start 88.138 101.346) (end 86.487 101.346) (width 0.25) (layer "B.Cu") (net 5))
 (segment (start 95.628 93.85) (end 94.3115 92.5335) (width 0.5) (layer "F.Cu") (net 30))
 (segment (start 95.625 91.22) (end 94.135 92.71) (width 0.5) (layer "F.Cu") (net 30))
 (segment (start 94.135 92.71) (end 93.345 92.71) (width 0.5) (layer "F.Cu") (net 30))
 (segment (start 95.625 90.17) (end 95.625 91.22) (width 0.5) (layer "F.Cu") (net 30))
 (segment (start 95.628 95.123) (end 95.628 93.85) (width 0.5) (layer "F.Cu") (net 30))
 (segment (start 98.425 90.17) (end 101.346 90.17) (width 0.5) (layer "F.Cu") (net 29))
 (segment (start 98.235 106.163) (end 99.285 106.163) (width 0.25) (layer "F.Cu") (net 3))
 (segment (start 100.171 105.277) (end 100.171 101.505) (width 0.25) (layer "F.Cu") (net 3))
 (segment (start 100.171 101.505) (end 101.346 100.33) (width 0.25) (layer "F.Cu") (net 3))
 (segment (start 99.285 106.163) (end 100.171 105.277) (width 0.25) (layer "F.Cu") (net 3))
 (segment (start 102.521 104.045) (end 101.346 102.87) (width 0.25) (layer "F.Cu") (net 28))
 (segment (start 102.521 106.902) (end 102.521 104.045) (width 0.25) (layer "F.Cu") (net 28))
 (segment (start 102.489 106.934) (end 102.521 106.902) (width 0.25) (layer "F.Cu") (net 28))
 (segment (start 97.464 106.934) (end 102.489 106.934) (width 0.25) (layer "F.Cu") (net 28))
 (segment (start 96.785 107.613) (end 97.464 106.934) (width 0.25) (layer "F.Cu") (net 28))
 (segment (start 84.402 99.113) (end 83.058 100.457) (width 0.25) (layer "F.Cu") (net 15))
 (segment (start 91.185 99.113) (end 84.402 99.113) (width 0.25) (layer "F.Cu") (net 15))
 (segment (start 87.778 100.563) (end 89.735 100.563) (width 0.25) (layer "F.Cu") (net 16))
 (segment (start 87.249 101.092) (end 87.778 100.563) (width 0.25) (layer "F.Cu") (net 16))
 (segment (start 83.058 102.997) (end 84.328 104.267) (width 0.25) (layer "F.Cu") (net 16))
 (segment (start 86.106 104.267) (end 87.249 103.124) (width 0.25) (layer "F.Cu") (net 16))
 (segment (start 87.249 103.124) (end 87.249 101.092) (width 0.25) (layer "F.Cu") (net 16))
 (segment (start 84.328 104.267) (end 86.106 104.267) (width 0.25) (layer "F.Cu") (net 16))
 (segment (start 91.567 97.663) (end 91.985 98.081) (width 0.25) (layer "F.Cu") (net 14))
 (segment (start 84.323722 101.722722) (end 81.792278 101.722722) (width 0.25) (layer "F.Cu") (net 14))
 (segment (start 83.320556 97.663) (end 91.567 97.663) (width 0.25) (layer "F.Cu") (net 14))
 (segment (start 81.792278 99.191278) (end 83.320556 97.663) (width 0.25) (layer "F.Cu") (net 14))
 (segment (start 81.792278 101.722722) (end 81.792278 99.191278) (width 0.25) (layer "F.Cu") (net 14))
 (segment (start 85.598 102.997) (end 84.323722 101.722722) (width 0.25) (layer "F.Cu") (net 14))
 (segment (start 91.985 98.081) (end 91.985 99.113) (width 0.25) (layer "F.Cu") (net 14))
 (segment (start 91.985 102.526) (end 91.948 102.489) (width 0.25) (layer "F.Cu") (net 23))
 (segment (start 93.345 95.01) (end 93.345 96.265) (width 0.25) (layer "F.Cu") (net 23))
 (segment (start 91.985 107.613) (end 91.985 102.526) (width 0.25) (layer "F.Cu") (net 23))
 (segment (start 93.345 96.393) (end 92.583 97.155) (width 0.25) (layer "F.Cu") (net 23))
 (segment (start 93.345 96.265) (end 94.235 97.155) (width 0.25) (layer "F.Cu") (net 23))
 (segment (start 93.116 95.239) (end 93.345 95.01) (width 0.25) (layer "F.Cu") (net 23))
 (segment (start 93.345 96.265) (end 93.345 96.393) (width 0.25) (layer "F.Cu") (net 23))
 (via (at 92.583 97.155) (size 0.8) (drill 0.4) (layers "F.Cu" "B.Cu") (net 23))
 (via (at 91.948 102.489) (size 0.8) (drill 0.4) (layers "F.Cu" "B.Cu") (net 23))
 (segment (start 92.583 97.155) (end 92.583 101.854) (width 0.25) (layer "B.Cu") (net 23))
 (segment (start 92.583 101.854) (end 91.948 102.489) (width 0.25) (layer "B.Cu") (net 23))
 (segment (start 89.7105 110.109) (end 89.5835 110.236) (width 0.25) (layer "F.Cu") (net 31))
 (segment (start 90.869 109.855) (end 90.996 109.728) (width 0.25) (layer "F.Cu") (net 31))
 (segment (start 89.4565 109.855) (end 90.869 109.855) (width 0.25) (layer "F.Cu") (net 31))
 (segment (start 92.646 109.728) (end 92.785 109.589) (width 0.25) (layer "F.Cu") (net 24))
 (segment (start 92.785 109.589) (end 92.785 107.613) (width 0.25) (layer "F.Cu") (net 24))
 (segment (start 95.985 107.613) (end 95.985 108.538) (width 0.25) (layer "F.Cu") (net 27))
 (segment (start 96.286 108.839) (end 100.711 108.839) (width 0.25) (layer "F.Cu") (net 27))
 (segment (start 95.985 108.538) (end 96.286 108.839) (width 0.25) (layer "F.Cu") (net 27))
 (segment (start 100.711 108.839) (end 101.346 108.204) (width 0.25) (layer "F.Cu") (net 27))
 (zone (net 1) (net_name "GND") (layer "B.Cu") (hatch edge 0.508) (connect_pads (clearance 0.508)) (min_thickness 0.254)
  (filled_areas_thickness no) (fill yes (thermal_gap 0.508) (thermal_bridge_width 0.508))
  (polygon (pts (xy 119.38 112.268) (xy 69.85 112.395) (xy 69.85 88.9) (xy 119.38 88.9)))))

